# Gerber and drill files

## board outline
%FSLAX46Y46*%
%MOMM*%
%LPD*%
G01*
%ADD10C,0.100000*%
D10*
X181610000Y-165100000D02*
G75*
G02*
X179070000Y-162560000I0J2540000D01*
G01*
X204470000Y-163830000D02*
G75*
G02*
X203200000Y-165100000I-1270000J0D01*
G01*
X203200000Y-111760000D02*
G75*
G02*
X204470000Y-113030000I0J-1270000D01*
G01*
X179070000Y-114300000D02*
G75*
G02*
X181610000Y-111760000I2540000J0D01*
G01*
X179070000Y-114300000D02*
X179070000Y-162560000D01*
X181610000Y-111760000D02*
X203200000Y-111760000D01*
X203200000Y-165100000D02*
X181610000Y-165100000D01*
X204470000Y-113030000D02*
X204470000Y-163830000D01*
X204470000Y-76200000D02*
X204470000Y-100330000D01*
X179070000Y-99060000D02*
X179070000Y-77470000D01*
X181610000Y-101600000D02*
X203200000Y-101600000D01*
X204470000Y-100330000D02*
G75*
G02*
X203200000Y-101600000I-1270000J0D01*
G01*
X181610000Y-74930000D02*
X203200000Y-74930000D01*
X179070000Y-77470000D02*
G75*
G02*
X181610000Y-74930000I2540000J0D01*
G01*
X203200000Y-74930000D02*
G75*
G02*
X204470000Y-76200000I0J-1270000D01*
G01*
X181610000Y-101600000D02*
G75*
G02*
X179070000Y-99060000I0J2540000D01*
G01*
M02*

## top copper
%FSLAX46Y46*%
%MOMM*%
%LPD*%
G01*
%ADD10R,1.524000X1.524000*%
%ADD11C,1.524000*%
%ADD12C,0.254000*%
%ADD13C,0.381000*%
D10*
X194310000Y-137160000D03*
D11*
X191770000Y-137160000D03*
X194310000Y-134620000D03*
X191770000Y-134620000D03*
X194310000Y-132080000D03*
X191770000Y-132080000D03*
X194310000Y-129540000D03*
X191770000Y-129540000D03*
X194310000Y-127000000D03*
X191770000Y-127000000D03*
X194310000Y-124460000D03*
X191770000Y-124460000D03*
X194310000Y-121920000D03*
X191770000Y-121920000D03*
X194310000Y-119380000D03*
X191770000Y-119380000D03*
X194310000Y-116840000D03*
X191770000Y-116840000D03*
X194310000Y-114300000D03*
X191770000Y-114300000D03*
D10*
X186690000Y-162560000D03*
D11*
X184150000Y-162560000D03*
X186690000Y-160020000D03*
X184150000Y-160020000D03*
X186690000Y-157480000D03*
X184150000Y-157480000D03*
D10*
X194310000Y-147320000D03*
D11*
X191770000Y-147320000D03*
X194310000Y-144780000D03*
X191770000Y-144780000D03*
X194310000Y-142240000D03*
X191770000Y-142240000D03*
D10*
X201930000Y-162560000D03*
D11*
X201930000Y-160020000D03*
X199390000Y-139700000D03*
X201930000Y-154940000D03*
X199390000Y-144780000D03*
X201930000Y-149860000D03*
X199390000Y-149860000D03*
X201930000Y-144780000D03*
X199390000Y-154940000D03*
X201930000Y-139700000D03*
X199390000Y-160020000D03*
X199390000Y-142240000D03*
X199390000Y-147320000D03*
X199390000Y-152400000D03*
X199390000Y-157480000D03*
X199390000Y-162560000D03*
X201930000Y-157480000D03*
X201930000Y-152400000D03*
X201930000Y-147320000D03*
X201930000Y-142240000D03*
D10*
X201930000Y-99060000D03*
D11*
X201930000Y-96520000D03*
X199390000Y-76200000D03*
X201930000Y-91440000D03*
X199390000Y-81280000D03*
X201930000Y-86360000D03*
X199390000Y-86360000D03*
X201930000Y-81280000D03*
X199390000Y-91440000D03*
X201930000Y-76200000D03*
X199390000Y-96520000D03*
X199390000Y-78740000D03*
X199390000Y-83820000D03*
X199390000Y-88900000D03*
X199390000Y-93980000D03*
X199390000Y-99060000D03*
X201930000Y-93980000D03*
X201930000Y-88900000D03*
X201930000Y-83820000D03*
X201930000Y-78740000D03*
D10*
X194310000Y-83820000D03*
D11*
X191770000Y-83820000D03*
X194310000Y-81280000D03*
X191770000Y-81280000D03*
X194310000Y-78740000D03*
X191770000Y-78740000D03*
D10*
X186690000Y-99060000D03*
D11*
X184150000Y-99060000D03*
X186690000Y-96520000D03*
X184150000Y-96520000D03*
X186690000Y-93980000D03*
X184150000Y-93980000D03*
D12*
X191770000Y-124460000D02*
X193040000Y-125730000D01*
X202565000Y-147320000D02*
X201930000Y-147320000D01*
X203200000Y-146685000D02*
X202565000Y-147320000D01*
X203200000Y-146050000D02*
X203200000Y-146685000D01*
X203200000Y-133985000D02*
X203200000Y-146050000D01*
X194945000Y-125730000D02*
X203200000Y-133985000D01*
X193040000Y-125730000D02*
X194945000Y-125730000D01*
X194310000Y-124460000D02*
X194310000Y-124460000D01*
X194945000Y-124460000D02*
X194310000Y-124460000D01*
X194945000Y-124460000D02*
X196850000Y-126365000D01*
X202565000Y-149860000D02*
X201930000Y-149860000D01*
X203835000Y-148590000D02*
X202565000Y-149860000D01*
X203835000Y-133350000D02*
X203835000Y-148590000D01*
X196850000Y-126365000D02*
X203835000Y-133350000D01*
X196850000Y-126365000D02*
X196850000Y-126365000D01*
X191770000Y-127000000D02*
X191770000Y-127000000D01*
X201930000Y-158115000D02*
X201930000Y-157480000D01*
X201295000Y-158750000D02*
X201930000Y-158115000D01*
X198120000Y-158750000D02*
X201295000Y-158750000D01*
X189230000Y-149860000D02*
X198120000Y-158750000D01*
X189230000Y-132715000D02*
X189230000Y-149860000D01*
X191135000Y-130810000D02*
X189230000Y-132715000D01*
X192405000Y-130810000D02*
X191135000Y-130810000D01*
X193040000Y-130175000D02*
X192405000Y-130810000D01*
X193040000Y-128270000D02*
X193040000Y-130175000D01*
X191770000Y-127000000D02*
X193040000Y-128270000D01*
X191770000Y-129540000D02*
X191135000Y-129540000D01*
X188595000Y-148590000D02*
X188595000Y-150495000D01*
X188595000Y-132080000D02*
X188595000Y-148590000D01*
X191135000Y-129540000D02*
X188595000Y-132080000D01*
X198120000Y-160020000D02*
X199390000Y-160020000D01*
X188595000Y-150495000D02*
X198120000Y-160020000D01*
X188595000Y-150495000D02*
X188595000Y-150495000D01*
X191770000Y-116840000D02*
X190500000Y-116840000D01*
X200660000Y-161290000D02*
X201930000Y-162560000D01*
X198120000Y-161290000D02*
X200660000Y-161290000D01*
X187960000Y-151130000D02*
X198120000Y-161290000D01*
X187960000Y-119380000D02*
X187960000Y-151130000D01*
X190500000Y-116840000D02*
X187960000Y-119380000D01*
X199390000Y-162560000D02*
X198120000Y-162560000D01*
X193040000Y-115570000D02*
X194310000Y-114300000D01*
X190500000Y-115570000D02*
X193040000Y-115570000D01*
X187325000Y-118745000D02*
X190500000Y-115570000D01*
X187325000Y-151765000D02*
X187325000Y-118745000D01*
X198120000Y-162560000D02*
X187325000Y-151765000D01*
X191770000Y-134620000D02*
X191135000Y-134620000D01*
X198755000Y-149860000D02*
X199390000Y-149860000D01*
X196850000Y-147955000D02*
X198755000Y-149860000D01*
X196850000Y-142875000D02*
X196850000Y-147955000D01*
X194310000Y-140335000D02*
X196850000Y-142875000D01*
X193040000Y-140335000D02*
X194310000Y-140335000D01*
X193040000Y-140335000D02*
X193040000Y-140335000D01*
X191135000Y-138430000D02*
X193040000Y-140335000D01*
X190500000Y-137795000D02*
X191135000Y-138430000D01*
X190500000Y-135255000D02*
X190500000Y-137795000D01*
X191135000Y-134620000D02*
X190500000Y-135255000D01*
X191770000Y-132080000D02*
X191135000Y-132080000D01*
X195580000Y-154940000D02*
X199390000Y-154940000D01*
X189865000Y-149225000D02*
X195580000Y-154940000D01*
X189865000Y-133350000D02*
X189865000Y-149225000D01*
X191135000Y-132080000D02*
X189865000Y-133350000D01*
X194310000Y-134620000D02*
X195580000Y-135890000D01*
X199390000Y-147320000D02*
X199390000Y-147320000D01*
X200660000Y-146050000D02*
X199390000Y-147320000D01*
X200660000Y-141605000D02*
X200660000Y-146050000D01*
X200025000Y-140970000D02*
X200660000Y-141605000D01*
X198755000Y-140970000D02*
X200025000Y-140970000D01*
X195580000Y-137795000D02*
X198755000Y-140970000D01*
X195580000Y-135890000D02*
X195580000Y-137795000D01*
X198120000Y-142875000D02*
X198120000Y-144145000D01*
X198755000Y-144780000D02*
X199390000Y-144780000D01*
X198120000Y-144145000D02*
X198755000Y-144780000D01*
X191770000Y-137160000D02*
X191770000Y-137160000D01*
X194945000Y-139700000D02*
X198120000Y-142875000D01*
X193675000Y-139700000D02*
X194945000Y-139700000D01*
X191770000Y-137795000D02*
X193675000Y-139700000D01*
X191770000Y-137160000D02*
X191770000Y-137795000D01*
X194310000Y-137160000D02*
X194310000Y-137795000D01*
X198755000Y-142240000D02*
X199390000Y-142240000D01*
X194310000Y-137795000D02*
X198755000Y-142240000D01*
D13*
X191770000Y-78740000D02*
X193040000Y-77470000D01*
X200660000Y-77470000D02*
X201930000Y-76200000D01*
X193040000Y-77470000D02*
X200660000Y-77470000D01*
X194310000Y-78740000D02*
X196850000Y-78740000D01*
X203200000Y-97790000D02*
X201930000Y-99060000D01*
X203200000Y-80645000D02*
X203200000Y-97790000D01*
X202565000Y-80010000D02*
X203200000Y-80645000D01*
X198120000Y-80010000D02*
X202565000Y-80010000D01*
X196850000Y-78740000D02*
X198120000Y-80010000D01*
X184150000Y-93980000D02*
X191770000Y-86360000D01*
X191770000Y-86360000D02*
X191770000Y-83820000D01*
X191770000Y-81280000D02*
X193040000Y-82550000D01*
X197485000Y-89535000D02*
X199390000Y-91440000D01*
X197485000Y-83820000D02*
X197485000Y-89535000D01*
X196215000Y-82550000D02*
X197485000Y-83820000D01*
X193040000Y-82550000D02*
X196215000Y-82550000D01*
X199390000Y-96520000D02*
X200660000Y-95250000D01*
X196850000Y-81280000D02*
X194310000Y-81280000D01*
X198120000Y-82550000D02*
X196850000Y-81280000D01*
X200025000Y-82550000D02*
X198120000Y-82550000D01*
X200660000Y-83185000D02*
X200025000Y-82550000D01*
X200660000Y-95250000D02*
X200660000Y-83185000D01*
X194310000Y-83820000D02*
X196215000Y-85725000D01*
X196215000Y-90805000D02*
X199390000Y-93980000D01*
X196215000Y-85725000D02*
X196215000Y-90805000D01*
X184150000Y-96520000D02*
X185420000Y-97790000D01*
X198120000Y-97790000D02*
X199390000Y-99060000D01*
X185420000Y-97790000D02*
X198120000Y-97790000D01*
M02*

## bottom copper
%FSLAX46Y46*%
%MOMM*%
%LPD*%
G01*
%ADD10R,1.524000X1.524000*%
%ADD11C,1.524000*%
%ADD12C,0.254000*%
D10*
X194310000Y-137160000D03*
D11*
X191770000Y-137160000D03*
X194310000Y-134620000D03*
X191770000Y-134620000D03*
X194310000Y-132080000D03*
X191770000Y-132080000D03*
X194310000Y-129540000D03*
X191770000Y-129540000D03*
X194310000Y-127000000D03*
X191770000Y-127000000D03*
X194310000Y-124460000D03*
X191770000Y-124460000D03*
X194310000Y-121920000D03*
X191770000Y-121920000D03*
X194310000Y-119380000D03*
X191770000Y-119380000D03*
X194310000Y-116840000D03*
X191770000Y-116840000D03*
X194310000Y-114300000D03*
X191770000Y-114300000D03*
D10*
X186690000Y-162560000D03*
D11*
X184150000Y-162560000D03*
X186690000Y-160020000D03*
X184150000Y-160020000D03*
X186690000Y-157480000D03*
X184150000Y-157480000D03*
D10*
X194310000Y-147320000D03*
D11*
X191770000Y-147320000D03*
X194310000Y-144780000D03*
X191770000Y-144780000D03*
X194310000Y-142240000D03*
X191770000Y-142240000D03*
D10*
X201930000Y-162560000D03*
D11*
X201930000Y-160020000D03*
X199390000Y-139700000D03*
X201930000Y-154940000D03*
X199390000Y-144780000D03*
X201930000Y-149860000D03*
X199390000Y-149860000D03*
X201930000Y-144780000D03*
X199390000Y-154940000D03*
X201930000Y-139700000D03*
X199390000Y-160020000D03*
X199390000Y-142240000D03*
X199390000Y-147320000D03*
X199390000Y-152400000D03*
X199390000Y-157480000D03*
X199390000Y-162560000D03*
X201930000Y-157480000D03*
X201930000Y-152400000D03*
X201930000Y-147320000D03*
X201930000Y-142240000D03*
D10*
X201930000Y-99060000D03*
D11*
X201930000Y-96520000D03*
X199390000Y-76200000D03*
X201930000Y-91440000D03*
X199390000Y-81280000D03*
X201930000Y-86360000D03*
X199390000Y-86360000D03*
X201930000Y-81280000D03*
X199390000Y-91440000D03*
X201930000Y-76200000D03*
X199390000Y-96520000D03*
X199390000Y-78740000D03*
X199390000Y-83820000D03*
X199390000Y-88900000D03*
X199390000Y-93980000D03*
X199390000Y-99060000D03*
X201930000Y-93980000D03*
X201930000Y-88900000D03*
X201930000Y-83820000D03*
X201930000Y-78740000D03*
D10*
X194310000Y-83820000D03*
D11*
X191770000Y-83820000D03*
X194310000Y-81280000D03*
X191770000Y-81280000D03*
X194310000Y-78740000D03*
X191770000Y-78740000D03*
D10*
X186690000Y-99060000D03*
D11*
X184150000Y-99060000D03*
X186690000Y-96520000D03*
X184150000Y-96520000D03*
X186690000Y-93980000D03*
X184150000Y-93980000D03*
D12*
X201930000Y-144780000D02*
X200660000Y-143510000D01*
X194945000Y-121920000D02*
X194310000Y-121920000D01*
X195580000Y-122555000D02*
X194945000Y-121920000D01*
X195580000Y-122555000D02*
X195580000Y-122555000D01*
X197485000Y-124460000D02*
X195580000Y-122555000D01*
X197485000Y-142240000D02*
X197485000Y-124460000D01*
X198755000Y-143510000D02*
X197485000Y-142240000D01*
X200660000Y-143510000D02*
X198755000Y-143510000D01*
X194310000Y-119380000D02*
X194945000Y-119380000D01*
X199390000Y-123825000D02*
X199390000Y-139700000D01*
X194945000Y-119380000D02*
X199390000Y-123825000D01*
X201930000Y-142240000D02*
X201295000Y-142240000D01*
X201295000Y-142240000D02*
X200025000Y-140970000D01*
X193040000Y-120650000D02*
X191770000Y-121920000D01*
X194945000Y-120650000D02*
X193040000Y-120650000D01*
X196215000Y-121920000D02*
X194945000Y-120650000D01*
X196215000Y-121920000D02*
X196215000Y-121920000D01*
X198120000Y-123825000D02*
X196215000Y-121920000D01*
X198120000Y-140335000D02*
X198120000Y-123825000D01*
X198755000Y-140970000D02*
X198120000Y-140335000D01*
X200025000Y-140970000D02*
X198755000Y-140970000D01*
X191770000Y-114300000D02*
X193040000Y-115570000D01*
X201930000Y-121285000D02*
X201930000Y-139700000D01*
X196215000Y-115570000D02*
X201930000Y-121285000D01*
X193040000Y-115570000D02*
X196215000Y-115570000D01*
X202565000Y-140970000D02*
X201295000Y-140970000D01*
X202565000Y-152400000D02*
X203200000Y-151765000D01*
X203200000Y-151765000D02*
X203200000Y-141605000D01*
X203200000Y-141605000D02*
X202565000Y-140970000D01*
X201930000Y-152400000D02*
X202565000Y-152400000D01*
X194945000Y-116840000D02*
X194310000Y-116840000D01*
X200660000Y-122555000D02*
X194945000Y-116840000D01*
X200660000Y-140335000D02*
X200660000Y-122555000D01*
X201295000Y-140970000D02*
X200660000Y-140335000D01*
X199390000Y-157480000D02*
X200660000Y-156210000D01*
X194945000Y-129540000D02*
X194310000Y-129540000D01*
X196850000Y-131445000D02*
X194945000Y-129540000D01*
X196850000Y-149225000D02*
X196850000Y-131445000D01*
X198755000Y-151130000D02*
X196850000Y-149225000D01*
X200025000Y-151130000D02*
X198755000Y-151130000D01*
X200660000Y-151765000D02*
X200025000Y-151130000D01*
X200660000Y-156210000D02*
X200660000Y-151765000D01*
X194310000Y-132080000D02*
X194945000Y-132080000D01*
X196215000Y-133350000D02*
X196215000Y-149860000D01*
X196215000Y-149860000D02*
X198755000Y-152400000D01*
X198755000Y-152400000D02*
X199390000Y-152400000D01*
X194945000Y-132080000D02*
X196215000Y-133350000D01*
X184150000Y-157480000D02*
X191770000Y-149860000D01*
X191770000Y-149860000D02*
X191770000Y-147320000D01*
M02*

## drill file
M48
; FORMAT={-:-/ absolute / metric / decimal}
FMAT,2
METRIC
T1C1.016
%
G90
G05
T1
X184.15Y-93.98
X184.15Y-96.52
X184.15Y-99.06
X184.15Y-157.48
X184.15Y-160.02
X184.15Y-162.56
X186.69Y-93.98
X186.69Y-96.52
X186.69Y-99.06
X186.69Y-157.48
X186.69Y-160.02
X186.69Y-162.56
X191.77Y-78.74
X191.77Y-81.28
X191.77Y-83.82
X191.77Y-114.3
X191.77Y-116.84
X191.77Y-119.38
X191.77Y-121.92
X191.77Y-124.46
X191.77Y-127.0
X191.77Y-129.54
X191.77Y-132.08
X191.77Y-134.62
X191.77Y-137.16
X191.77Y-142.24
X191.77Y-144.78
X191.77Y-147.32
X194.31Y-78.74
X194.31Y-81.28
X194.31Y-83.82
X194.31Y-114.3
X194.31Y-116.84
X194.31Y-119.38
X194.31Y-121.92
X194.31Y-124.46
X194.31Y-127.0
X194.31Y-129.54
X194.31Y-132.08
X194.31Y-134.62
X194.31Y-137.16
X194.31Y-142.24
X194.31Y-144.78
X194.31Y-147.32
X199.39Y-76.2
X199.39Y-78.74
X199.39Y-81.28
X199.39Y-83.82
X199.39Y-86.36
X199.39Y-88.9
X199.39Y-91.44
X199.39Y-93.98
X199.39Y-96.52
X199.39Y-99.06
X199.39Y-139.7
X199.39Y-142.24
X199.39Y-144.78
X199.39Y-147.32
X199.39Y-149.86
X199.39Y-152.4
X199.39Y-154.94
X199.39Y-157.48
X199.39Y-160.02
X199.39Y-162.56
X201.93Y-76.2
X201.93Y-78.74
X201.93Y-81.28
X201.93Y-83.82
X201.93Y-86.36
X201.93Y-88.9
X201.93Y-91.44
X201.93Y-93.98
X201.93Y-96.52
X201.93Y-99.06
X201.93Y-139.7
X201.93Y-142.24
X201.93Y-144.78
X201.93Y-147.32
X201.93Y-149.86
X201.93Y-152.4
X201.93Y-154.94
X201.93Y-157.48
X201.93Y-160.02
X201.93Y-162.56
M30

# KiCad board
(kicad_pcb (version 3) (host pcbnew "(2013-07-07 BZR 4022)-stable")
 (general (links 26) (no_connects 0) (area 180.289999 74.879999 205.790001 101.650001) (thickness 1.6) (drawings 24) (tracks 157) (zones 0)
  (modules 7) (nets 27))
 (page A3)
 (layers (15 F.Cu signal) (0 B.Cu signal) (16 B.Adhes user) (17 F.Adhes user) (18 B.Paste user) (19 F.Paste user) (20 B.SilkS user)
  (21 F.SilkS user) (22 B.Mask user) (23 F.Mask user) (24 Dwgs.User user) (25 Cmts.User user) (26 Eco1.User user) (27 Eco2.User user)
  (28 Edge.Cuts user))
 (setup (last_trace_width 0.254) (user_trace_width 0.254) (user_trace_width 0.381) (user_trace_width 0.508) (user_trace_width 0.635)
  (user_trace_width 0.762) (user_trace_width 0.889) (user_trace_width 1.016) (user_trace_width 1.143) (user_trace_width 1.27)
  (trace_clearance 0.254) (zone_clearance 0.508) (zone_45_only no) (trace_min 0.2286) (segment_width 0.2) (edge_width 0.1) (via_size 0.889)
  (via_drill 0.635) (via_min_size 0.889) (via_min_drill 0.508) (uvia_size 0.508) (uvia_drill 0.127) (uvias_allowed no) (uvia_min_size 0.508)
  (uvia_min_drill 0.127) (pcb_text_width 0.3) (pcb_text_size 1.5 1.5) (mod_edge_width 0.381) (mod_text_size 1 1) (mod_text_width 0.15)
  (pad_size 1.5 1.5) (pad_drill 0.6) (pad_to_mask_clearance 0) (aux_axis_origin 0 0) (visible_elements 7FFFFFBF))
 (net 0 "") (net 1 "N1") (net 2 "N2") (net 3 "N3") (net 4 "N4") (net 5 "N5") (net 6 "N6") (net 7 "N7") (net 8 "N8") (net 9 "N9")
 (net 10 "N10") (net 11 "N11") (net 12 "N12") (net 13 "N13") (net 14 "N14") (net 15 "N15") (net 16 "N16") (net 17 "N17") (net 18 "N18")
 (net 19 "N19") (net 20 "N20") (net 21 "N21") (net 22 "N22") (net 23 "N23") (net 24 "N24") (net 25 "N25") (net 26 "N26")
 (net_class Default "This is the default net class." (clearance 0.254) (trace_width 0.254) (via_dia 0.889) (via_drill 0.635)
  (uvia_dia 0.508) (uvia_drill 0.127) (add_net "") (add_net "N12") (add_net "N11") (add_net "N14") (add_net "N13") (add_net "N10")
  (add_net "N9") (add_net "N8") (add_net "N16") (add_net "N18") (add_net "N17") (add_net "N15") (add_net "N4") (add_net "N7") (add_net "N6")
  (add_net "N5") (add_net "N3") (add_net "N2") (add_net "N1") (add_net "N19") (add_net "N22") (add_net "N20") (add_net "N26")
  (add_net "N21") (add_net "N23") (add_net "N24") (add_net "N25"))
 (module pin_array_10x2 (layer F.Cu) (at 193.04 125.73 90)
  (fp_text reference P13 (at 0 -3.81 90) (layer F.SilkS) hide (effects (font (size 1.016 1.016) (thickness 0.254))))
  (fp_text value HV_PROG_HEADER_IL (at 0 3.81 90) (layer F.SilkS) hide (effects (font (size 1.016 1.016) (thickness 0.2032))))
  (pad 1 thru_hole rect (at -11.43 1.27 90) (size 1.524 1.524) (drill 1.016) (layers *.Cu *.Mask F.SilkS) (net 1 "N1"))
  (pad 2 thru_hole circle (at -11.43 -1.27 90) (size 1.524 1.524) (drill 1.016) (layers *.Cu *.Mask F.SilkS) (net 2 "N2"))
  (pad 3 thru_hole circle (at -8.89 1.27 90) (size 1.524 1.524) (drill 1.016) (layers *.Cu *.Mask F.SilkS) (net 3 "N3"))
  (pad 4 thru_hole circle (at -8.89 -1.27 90) (size 1.524 1.524) (drill 1.016) (layers *.Cu *.Mask F.SilkS) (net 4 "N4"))
  (pad 5 thru_hole circle (at -6.35 1.27 90) (size 1.524 1.524) (drill 1.016) (layers *.Cu *.Mask F.SilkS) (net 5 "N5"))
  (pad 6 thru_hole circle (at -6.35 -1.27 90) (size 1.524 1.524) (drill 1.016) (layers *.Cu *.Mask F.SilkS) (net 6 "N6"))
  (pad 7 thru_hole circle (at -3.81 1.27 90) (size 1.524 1.524) (drill 1.016) (layers *.Cu *.Mask F.SilkS) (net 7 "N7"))
  (pad 8 thru_hole circle (at -3.81 -1.27 90) (size 1.524 1.524) (drill 1.016) (layers *.Cu *.Mask F.SilkS) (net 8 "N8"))
  (pad 9 thru_hole circle (at -1.27 1.27 90) (size 1.524 1.524) (drill 1.016) (layers *.Cu *.Mask F.SilkS))
  (pad 10 thru_hole circle (at -1.27 -1.27 90) (size 1.524 1.524) (drill 1.016) (layers *.Cu *.Mask F.SilkS) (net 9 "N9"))
  (pad 11 thru_hole circle (at 1.27 1.27 90) (size 1.524 1.524) (drill 1.016) (layers *.Cu *.Mask F.SilkS) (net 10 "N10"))
  (pad 12 thru_hole circle (at 1.27 -1.27 90) (size 1.524 1.524) (drill 1.016) (layers *.Cu *.Mask F.SilkS) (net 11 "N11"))
  (pad 13 thru_hole circle (at 3.81 1.27 90) (size 1.524 1.524) (drill 1.016) (layers *.Cu *.Mask F.SilkS) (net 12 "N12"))
  (pad 14 thru_hole circle (at 3.81 -1.27 90) (size 1.524 1.524) (drill 1.016) (layers *.Cu *.Mask F.SilkS) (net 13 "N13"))
  (pad 15 thru_hole circle (at 6.35 1.27 90) (size 1.524 1.524) (drill 1.016) (layers *.Cu *.Mask F.SilkS) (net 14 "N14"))
  (pad 16 thru_hole circle (at 6.35 -1.27 90) (size 1.524 1.524) (drill 1.016) (layers *.Cu *.Mask F.SilkS))
  (pad 17 thru_hole circle (at 8.89 1.27 90) (size 1.524 1.524) (drill 1.016) (layers *.Cu *.Mask F.SilkS) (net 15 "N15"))
  (pad 18 thru_hole circle (at 8.89 -1.27 90) (size 1.524 1.524) (drill 1.016) (layers *.Cu *.Mask F.SilkS) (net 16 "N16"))
  (pad 19 thru_hole circle (at 11.43 1.27 90) (size 1.524 1.524) (drill 1.016) (layers *.Cu *.Mask F.SilkS) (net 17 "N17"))
  (pad 20 thru_hole circle (at 11.43 -1.27 90) (size 1.524 1.524) (drill 1.016) (layers *.Cu *.Mask F.SilkS) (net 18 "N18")))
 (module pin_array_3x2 (layer F.Cu) (at 185.42 160.02 90)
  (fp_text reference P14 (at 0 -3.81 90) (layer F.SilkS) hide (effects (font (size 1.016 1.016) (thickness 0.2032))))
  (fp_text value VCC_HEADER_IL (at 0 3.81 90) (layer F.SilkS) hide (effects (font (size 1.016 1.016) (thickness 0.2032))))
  (pad 1 thru_hole rect (at -2.54 1.27 90) (size 1.524 1.524) (drill 1.016) (layers *.Cu *.Mask F.SilkS))
  (pad 2 thru_hole circle (at -2.54 -1.27 90) (size 1.524 1.524) (drill 1.016) (layers *.Cu *.Mask F.SilkS))
  (pad 3 thru_hole circle (at 0 1.27 90) (size 1.524 1.524) (drill 1.016) (layers *.Cu *.Mask F.SilkS))
  (pad 4 thru_hole circle (at 0 -1.27 90) (size 1.524 1.524) (drill 1.016) (layers *.Cu *.Mask F.SilkS))
  (pad 5 thru_hole circle (at 2.54 1.27 90) (size 1.524 1.524) (drill 1.016) (layers *.Cu *.Mask F.SilkS))
  (pad 6 thru_hole circle (at 2.54 -1.27 90) (size 1.524 1.524) (drill 1.016) (layers *.Cu *.Mask F.SilkS) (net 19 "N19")))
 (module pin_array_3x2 (layer F.Cu) (at 193.04 144.78 90)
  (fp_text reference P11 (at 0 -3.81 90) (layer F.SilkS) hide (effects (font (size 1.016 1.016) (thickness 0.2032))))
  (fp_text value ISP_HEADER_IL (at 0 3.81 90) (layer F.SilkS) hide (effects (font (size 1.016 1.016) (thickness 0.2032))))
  (pad 1 thru_hole rect (at -2.54 1.27 90) (size 1.524 1.524) (drill 1.016) (layers *.Cu *.Mask F.SilkS))
  (pad 2 thru_hole circle (at -2.54 -1.27 90) (size 1.524 1.524) (drill 1.016) (layers *.Cu *.Mask F.SilkS) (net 19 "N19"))
  (pad 3 thru_hole circle (at 0 1.27 90) (size 1.524 1.524) (drill 1.016) (layers *.Cu *.Mask F.SilkS))
  (pad 4 thru_hole circle (at 0 -1.27 90) (size 1.524 1.524) (drill 1.016) (layers *.Cu *.Mask F.SilkS))
  (pad 5 thru_hole circle (at 2.54 1.27 90) (size 1.524 1.524) (drill 1.016) (layers *.Cu *.Mask F.SilkS))
  (pad 6 thru_hole circle (at 2.54 -1.27 90) (size 1.524 1.524) (drill 1.016) (layers *.Cu *.Mask F.SilkS)))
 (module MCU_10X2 (layer F.Cu) (at 200.66 151.13 90)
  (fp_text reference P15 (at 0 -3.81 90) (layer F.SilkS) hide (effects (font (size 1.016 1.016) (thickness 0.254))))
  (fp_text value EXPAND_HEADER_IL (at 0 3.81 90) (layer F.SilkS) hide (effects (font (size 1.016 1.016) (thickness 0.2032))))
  (pad 1 thru_hole rect (at -11.43 1.27 90) (size 1.524 1.524) (drill 1.016) (layers *.Cu *.Mask F.SilkS) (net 16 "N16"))
  (pad 2 thru_hole circle (at -8.89 1.27 90) (size 1.524 1.524) (drill 1.016) (layers *.Cu *.Mask F.SilkS))
  (pad 11 thru_hole circle (at 11.43 -1.27 90) (size 1.524 1.524) (drill 1.016) (layers *.Cu *.Mask F.SilkS) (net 14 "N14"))
  (pad 4 thru_hole circle (at -3.81 1.27 90) (size 1.524 1.524) (drill 1.016) (layers *.Cu *.Mask F.SilkS))
  (pad 13 thru_hole circle (at 6.35 -1.27 90) (size 1.524 1.524) (drill 1.016) (layers *.Cu *.Mask F.SilkS) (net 2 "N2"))
  (pad 6 thru_hole circle (at 1.27 1.27 90) (size 1.524 1.524) (drill 1.016) (layers *.Cu *.Mask F.SilkS) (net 10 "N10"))
  (pad 15 thru_hole circle (at 1.27 -1.27 90) (size 1.524 1.524) (drill 1.016) (layers *.Cu *.Mask F.SilkS) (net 4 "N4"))
  (pad 8 thru_hole circle (at 6.35 1.27 90) (size 1.524 1.524) (drill 1.016) (layers *.Cu *.Mask F.SilkS) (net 12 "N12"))
  (pad 17 thru_hole circle (at -3.81 -1.27 90) (size 1.524 1.524) (drill 1.016) (layers *.Cu *.Mask F.SilkS) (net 6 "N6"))
  (pad 10 thru_hole circle (at 11.43 1.27 90) (size 1.524 1.524) (drill 1.016) (layers *.Cu *.Mask F.SilkS) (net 18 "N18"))
  (pad 19 thru_hole circle (at -8.89 -1.27 90) (size 1.524 1.524) (drill 1.016) (layers *.Cu *.Mask F.SilkS) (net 8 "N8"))
  (pad 12 thru_hole circle (at 8.89 -1.27 90) (size 1.524 1.524) (drill 1.016) (layers *.Cu *.Mask F.SilkS) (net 1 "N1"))
  (pad 14 thru_hole circle (at 3.81 -1.27 90) (size 1.524 1.524) (drill 1.016) (layers *.Cu *.Mask F.SilkS) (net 3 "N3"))
  (pad 16 thru_hole circle (at -1.27 -1.27 90) (size 1.524 1.524) (drill 1.016) (layers *.Cu *.Mask F.SilkS) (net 5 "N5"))
  (pad 18 thru_hole circle (at -6.35 -1.27 90) (size 1.524 1.524) (drill 1.016) (layers *.Cu *.Mask F.SilkS) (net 7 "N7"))
  (pad 20 thru_hole circle (at -11.43 -1.27 90) (size 1.524 1.524) (drill 1.016) (layers *.Cu *.Mask F.SilkS) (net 17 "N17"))
  (pad 3 thru_hole circle (at -6.35 1.27 90) (size 1.524 1.524) (drill 1.016) (layers *.Cu *.Mask F.SilkS) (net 9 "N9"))
  (pad 5 thru_hole circle (at -1.27 1.27 90) (size 1.524 1.524) (drill 1.016) (layers *.Cu *.Mask F.SilkS) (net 15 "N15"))
  (pad 7 thru_hole circle (at 3.81 1.27 90) (size 1.524 1.524) (drill 1.016) (layers *.Cu *.Mask F.SilkS) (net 11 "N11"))
  (pad 9 thru_hole circle (at 8.89 1.27 90) (size 1.524 1.524) (drill 1.016) (layers *.Cu *.Mask F.SilkS) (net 13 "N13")))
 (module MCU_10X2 (layer F.Cu) (at 200.66 87.63 90)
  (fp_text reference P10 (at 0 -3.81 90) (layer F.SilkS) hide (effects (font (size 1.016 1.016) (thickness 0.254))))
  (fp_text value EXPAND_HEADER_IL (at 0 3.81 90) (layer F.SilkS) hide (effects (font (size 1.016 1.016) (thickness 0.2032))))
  (pad 1 thru_hole rect (at -11.43 1.27 90) (size 1.524 1.524) (drill 1.016) (layers *.Cu *.Mask F.SilkS) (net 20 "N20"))
  (pad 2 thru_hole circle (at -8.89 1.27 90) (size 1.524 1.524) (drill 1.016) (layers *.Cu *.Mask F.SilkS))
  (pad 11 thru_hole circle (at 11.43 -1.27 90) (size 1.524 1.524) (drill 1.016) (layers *.Cu *.Mask F.SilkS))
  (pad 4 thru_hole circle (at -3.81 1.27 90) (size 1.524 1.524) (drill 1.016) (layers *.Cu *.Mask F.SilkS))
  (pad 13 thru_hole circle (at 6.35 -1.27 90) (size 1.524 1.524) (drill 1.016) (layers *.Cu *.Mask F.SilkS))
  (pad 6 thru_hole circle (at 1.27 1.27 90) (size 1.524 1.524) (drill 1.016) (layers *.Cu *.Mask F.SilkS))
  (pad 15 thru_hole circle (at 1.27 -1.27 90) (size 1.524 1.524) (drill 1.016) (layers *.Cu *.Mask F.SilkS))
  (pad 8 thru_hole circle (at 6.35 1.27 90) (size 1.524 1.524) (drill 1.016) (layers *.Cu *.Mask F.SilkS))
  (pad 17 thru_hole circle (at -3.81 -1.27 90) (size 1.524 1.524) (drill 1.016) (layers *.Cu *.Mask F.SilkS) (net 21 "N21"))
  (pad 10 thru_hole circle (at 11.43 1.27 90) (size 1.524 1.524) (drill 1.016) (layers *.Cu *.Mask F.SilkS) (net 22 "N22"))
  (pad 19 thru_hole circle (at -8.89 -1.27 90) (size 1.524 1.524) (drill 1.016) (layers *.Cu *.Mask F.SilkS) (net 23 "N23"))
  (pad 12 thru_hole circle (at 8.89 -1.27 90) (size 1.524 1.524) (drill 1.016) (layers *.Cu *.Mask F.SilkS))
  (pad 14 thru_hole circle (at 3.81 -1.27 90) (size 1.524 1.524) (drill 1.016) (layers *.Cu *.Mask F.SilkS))
  (pad 16 thru_hole circle (at -1.27 -1.27 90) (size 1.524 1.524) (drill 1.016) (layers *.Cu *.Mask F.SilkS))
  (pad 18 thru_hole circle (at -6.35 -1.27 90) (size 1.524 1.524) (drill 1.016) (layers *.Cu *.Mask F.SilkS) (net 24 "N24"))
  (pad 20 thru_hole circle (at -11.43 -1.27 90) (size 1.524 1.524) (drill 1.016) (layers *.Cu *.Mask F.SilkS) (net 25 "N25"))
  (pad 3 thru_hole circle (at -6.35 1.27 90) (size 1.524 1.524) (drill 1.016) (layers *.Cu *.Mask F.SilkS))
  (pad 5 thru_hole circle (at -1.27 1.27 90) (size 1.524 1.524) (drill 1.016) (layers *.Cu *.Mask F.SilkS))
  (pad 7 thru_hole circle (at 3.81 1.27 90) (size 1.524 1.524) (drill 1.016) (layers *.Cu *.Mask F.SilkS))
  (pad 9 thru_hole circle (at 8.89 1.27 90) (size 1.524 1.524) (drill 1.016) (layers *.Cu *.Mask F.SilkS)))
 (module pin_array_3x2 (layer F.Cu) (at 193.04 81.28 90)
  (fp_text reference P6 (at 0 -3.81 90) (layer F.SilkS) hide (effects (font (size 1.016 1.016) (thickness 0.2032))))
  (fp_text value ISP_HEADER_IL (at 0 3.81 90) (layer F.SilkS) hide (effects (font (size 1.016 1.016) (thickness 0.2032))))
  (pad 1 thru_hole rect (at -2.54 1.27 90) (size 1.524 1.524) (drill 1.016) (layers *.Cu *.Mask F.SilkS) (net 24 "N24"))
  (pad 2 thru_hole circle (at -2.54 -1.27 90) (size 1.524 1.524) (drill 1.016) (layers *.Cu *.Mask F.SilkS) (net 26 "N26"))
  (pad 3 thru_hole circle (at 0 1.27 90) (size 1.524 1.524) (drill 1.016) (layers *.Cu *.Mask F.SilkS) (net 23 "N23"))
  (pad 4 thru_hole circle (at 0 -1.27 90) (size 1.524 1.524) (drill 1.016) (layers *.Cu *.Mask F.SilkS) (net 21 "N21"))
  (pad 5 thru_hole circle (at 2.54 1.27 90) (size 1.524 1.524) (drill 1.016) (layers *.Cu *.Mask F.SilkS) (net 20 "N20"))
  (pad 6 thru_hole circle (at 2.54 -1.27 90) (size 1.524 1.524) (drill 1.016) (layers *.Cu *.Mask F.SilkS) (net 22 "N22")))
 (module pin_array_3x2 (layer F.Cu) (at 185.42 96.52 90)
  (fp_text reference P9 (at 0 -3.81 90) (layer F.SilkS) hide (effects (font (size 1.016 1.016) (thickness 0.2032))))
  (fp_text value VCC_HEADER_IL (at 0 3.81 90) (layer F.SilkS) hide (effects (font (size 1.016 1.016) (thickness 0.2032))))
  (pad 1 thru_hole rect (at -2.54 1.27 90) (size 1.524 1.524) (drill 1.016) (layers *.Cu *.Mask F.SilkS))
  (pad 2 thru_hole circle (at -2.54 -1.27 90) (size 1.524 1.524) (drill 1.016) (layers *.Cu *.Mask F.SilkS))
  (pad 3 thru_hole circle (at 0 1.27 90) (size 1.524 1.524) (drill 1.016) (layers *.Cu *.Mask F.SilkS))
  (pad 4 thru_hole circle (at 0 -1.27 90) (size 1.524 1.524) (drill 1.016) (layers *.Cu *.Mask F.SilkS) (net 25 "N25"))
  (pad 5 thru_hole circle (at 2.54 1.27 90) (size 1.524 1.524) (drill 1.016) (layers *.Cu *.Mask F.SilkS))
  (pad 6 thru_hole circle (at 2.54 -1.27 90) (size 1.524 1.524) (drill 1.016) (layers *.Cu *.Mask F.SilkS) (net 26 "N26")))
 (gr_arc (start 181.61 162.56) (end 181.61 165.1) (angle 90) (layer Edge.Cuts) (width 0.1))
 (gr_arc (start 203.2 163.83) (end 204.47 163.83) (angle 90) (layer Edge.Cuts) (width 0.1))
 (gr_arc (start 203.2 113.03) (end 203.2 111.76) (angle 90) (layer Edge.Cuts) (width 0.1))
 (gr_arc (start 181.61 114.3) (end 179.07 114.3) (angle 90) (layer Edge.Cuts) (width 0.1))
 (gr_line (start 179.07 114.3) (end 179.07 162.56) (angle 90) (layer Edge.Cuts) (width 0.1))
 (gr_line (start 181.61 111.76) (end 203.2 111.76) (angle 90) (layer Edge.Cuts) (width 0.1))
 (gr_line (start 203.2 165.1) (end 181.61 165.1) (angle 90) (layer Edge.Cuts) (width 0.1))
 (gr_line (start 204.47 113.03) (end 204.47 163.83) (angle 90) (layer Edge.Cuts) (width 0.1))
 (gr_line (start 204.47 76.2) (end 204.47 100.33) (angle 90) (layer Edge.Cuts) (width 0.1))
 (gr_line (start 179.07 99.06) (end 179.07 77.47) (angle 90) (layer Edge.Cuts) (width 0.1))
 (gr_line (start 181.61 101.6) (end 203.2 101.6) (angle 90) (layer Edge.Cuts) (width 0.1))
 (gr_arc (start 203.2 100.33) (end 204.47 100.33) (angle 90) (layer Edge.Cuts) (width 0.1))
 (gr_line (start 181.61 74.93) (end 203.2 74.93) (angle 90) (layer Edge.Cuts) (width 0.1))
 (gr_arc (start 181.61 77.47) (end 179.07 77.47) (angle 90) (layer Edge.Cuts) (width 0.1))
 (gr_arc (start 203.2 76.2) (end 203.2 74.93) (angle 90) (layer Edge.Cuts) (width 0.1))
 (gr_arc (start 181.61 99.06) (end 181.61 101.6) (angle 90) (layer Edge.Cuts) (width 0.1))
 (segment (start 201.93 144.78) (end 200.66 143.51) (width 0.254) (layer B.Cu) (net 12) (status 400000))
 (segment (start 194.945 121.92) (end 194.31 121.92) (width 0.254) (layer B.Cu) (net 12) (status C00000))
 (segment (start 195.58 122.555) (end 194.945 121.92) (width 0.254) (layer B.Cu) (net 12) (status 800000))
 (segment (start 195.58 122.555) (end 195.58 122.555) (width 0.254) (layer B.Cu) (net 12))
 (segment (start 197.485 124.46) (end 195.58 122.555) (width 0.254) (layer B.Cu) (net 12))
 (segment (start 197.485 142.24) (end 197.485 124.46) (width 0.254) (layer B.Cu) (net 12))
 (segment (start 198.755 143.51) (end 197.485 142.24) (width 0.254) (layer B.Cu) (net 12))
 (segment (start 200.66 143.51) (end 198.755 143.51) (width 0.254) (layer B.Cu) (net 12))
 (segment (start 191.77 124.46) (end 193.04 125.73) (width 0.254) (layer F.Cu) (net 11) (status 400000))
 (segment (start 202.565 147.32) (end 201.93 147.32) (width 0.254) (layer F.Cu) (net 11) (status C00000))
 (segment (start 203.2 146.685) (end 202.565 147.32) (width 0.254) (layer F.Cu) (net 11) (status 800000))
 (segment (start 203.2 146.05) (end 203.2 146.685) (width 0.254) (layer F.Cu) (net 11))
 (segment (start 203.2 133.985) (end 203.2 146.05) (width 0.254) (layer F.Cu) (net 11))
 (segment (start 194.945 125.73) (end 203.2 133.985) (width 0.254) (layer F.Cu) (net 11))
 (segment (start 193.04 125.73) (end 194.945 125.73) (width 0.254) (layer F.Cu) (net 11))
 (segment (start 194.31 119.38) (end 194.945 119.38) (width 0.254) (layer B.Cu) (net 14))
 (segment (start 199.39 123.825) (end 199.39 139.7) (width 0.254) (layer B.Cu) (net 14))
 (segment (start 194.945 119.38) (end 199.39 123.825) (width 0.254) (layer B.Cu) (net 14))
 (segment (start 201.93 142.24) (end 201.295 142.24) (width 0.254) (layer B.Cu) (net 13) (status C00000))
 (segment (start 201.295 142.24) (end 200.025 140.97) (width 0.254) (layer B.Cu) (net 13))
 (segment (start 193.04 120.65) (end 191.77 121.92) (width 0.254) (layer B.Cu) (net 13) (status 800000))
 (segment (start 194.945 120.65) (end 193.04 120.65) (width 0.254) (layer B.Cu) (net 13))
 (segment (start 196.215 121.92) (end 194.945 120.65) (width 0.254) (layer B.Cu) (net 13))
 (segment (start 196.215 121.92) (end 196.215 121.92) (width 0.254) (layer B.Cu) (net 13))
 (segment (start 198.12 123.825) (end 196.215 121.92) (width 0.254) (layer B.Cu) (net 13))
 (segment (start 198.12 140.335) (end 198.12 123.825) (width 0.254) (layer B.Cu) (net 13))
 (segment (start 198.755 140.97) (end 198.12 140.335) (width 0.254) (layer B.Cu) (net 13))
 (segment (start 200.025 140.97) (end 198.755 140.97) (width 0.254) (layer B.Cu) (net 13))
 (segment (start 194.31 124.46) (end 194.31 124.46) (width 0.254) (layer F.Cu) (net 10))
 (segment (start 194.945 124.46) (end 194.31 124.46) (width 0.254) (layer F.Cu) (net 10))
 (segment (start 194.945 124.46) (end 196.85 126.365) (width 0.254) (layer F.Cu) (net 10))
 (segment (start 202.565 149.86) (end 201.93 149.86) (width 0.254) (layer F.Cu) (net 10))
 (segment (start 203.835 148.59) (end 202.565 149.86) (width 0.254) (layer F.Cu) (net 10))
 (segment (start 203.835 133.35) (end 203.835 148.59) (width 0.254) (layer F.Cu) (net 10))
 (segment (start 196.85 126.365) (end 203.835 133.35) (width 0.254) (layer F.Cu) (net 10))
 (segment (start 196.85 126.365) (end 196.85 126.365) (width 0.254) (layer F.Cu) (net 10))
 (segment (start 191.77 127) (end 191.77 127) (width 0.254) (layer F.Cu) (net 9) (status C00000))
 (segment (start 201.93 158.115) (end 201.93 157.48) (width 0.254) (layer F.Cu) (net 9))
 (segment (start 201.295 158.75) (end 201.93 158.115) (width 0.254) (layer F.Cu) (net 9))
 (segment (start 198.12 158.75) (end 201.295 158.75) (width 0.254) (layer F.Cu) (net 9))
 (segment (start 189.23 149.86) (end 198.12 158.75) (width 0.254) (layer F.Cu) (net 9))
 (segment (start 189.23 132.715) (end 189.23 149.86) (width 0.254) (layer F.Cu) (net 9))
 (segment (start 191.135 130.81) (end 189.23 132.715) (width 0.254) (layer F.Cu) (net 9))
 (segment (start 192.405 130.81) (end 191.135 130.81) (width 0.254) (layer F.Cu) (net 9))
 (segment (start 193.04 130.175) (end 192.405 130.81) (width 0.254) (layer F.Cu) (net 9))
 (segment (start 193.04 128.27) (end 193.04 130.175) (width 0.254) (layer F.Cu) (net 9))
 (segment (start 191.77 127) (end 193.04 128.27) (width 0.254) (layer F.Cu) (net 9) (status 400000))
 (segment (start 191.77 129.54) (end 191.135 129.54) (width 0.254) (layer F.Cu) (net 8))
 (segment (start 188.595 148.59) (end 188.595 150.495) (width 0.254) (layer F.Cu) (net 8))
 (segment (start 188.595 132.08) (end 188.595 148.59) (width 0.254) (layer F.Cu) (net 8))
 (segment (start 191.135 129.54) (end 188.595 132.08) (width 0.254) (layer F.Cu) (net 8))
 (segment (start 198.12 160.02) (end 199.39 160.02) (width 0.254) (layer F.Cu) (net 8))
 (segment (start 188.595 150.495) (end 198.12 160.02) (width 0.254) (layer F.Cu) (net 8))
 (segment (start 188.595 150.495) (end 188.595 150.495) (width 0.254) (layer F.Cu) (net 8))
 (segment (start 191.77 116.84) (end 190.5 116.84) (width 0.254) (layer F.Cu) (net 16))
 (segment (start 200.66 161.29) (end 201.93 162.56) (width 0.254) (layer F.Cu) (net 16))
 (segment (start 198.12 161.29) (end 200.66 161.29) (width 0.254) (layer F.Cu) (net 16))
 (segment (start 187.96 151.13) (end 198.12 161.29) (width 0.254) (layer F.Cu) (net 16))
 (segment (start 187.96 119.38) (end 187.96 151.13) (width 0.254) (layer F.Cu) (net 16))
 (segment (start 190.5 116.84) (end 187.96 119.38) (width 0.254) (layer F.Cu) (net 16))
 (segment (start 191.77 114.3) (end 193.04 115.57) (width 0.254) (layer B.Cu) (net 18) (status 400000))
 (segment (start 201.93 121.285) (end 201.93 139.7) (width 0.254) (layer B.Cu) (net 18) (status 800000))
 (segment (start 196.215 115.57) (end 201.93 121.285) (width 0.254) (layer B.Cu) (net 18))
 (segment (start 193.04 115.57) (end 196.215 115.57) (width 0.254) (layer B.Cu) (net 18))
 (segment (start 199.39 162.56) (end 198.12 162.56) (width 0.254) (layer F.Cu) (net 17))
 (segment (start 193.04 115.57) (end 194.31 114.3) (width 0.254) (layer F.Cu) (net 17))
 (segment (start 190.5 115.57) (end 193.04 115.57) (width 0.254) (layer F.Cu) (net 17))
 (segment (start 187.325 118.745) (end 190.5 115.57) (width 0.254) (layer F.Cu) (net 17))
 (segment (start 187.325 151.765) (end 187.325 118.745) (width 0.254) (layer F.Cu) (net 17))
 (segment (start 198.12 162.56) (end 187.325 151.765) (width 0.254) (layer F.Cu) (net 17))
 (segment (start 202.565 140.97) (end 201.295 140.97) (width 0.254) (layer B.Cu) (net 15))
 (segment (start 202.565 152.4) (end 203.2 151.765) (width 0.254) (layer B.Cu) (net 15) (status 400000))
 (segment (start 203.2 151.765) (end 203.2 141.605) (width 0.254) (layer B.Cu) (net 15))
 (segment (start 203.2 141.605) (end 202.565 140.97) (width 0.254) (layer B.Cu) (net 15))
 (segment (start 201.93 152.4) (end 202.565 152.4) (width 0.254) (layer B.Cu) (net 15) (status C00000))
 (segment (start 194.945 116.84) (end 194.31 116.84) (width 0.254) (layer B.Cu) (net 15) (status C00000))
 (segment (start 200.66 122.555) (end 194.945 116.84) (width 0.254) (layer B.Cu) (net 15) (status 800000))
 (segment (start 200.66 140.335) (end 200.66 122.555) (width 0.254) (layer B.Cu) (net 15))
 (segment (start 201.295 140.97) (end 200.66 140.335) (width 0.254) (layer B.Cu) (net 15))
 (segment (start 191.77 134.62) (end 191.135 134.62) (width 0.254) (layer F.Cu) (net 4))
 (segment (start 198.755 149.86) (end 199.39 149.86) (width 0.254) (layer F.Cu) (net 4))
 (segment (start 196.85 147.955) (end 198.755 149.86) (width 0.254) (layer F.Cu) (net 4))
 (segment (start 196.85 142.875) (end 196.85 147.955) (width 0.254) (layer F.Cu) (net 4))
 (segment (start 194.31 140.335) (end 196.85 142.875) (width 0.254) (layer F.Cu) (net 4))
 (segment (start 193.04 140.335) (end 194.31 140.335) (width 0.254) (layer F.Cu) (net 4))
 (segment (start 193.04 140.335) (end 193.04 140.335) (width 0.254) (layer F.Cu) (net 4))
 (segment (start 191.135 138.43) (end 193.04 140.335) (width 0.254) (layer F.Cu) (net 4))
 (segment (start 190.5 137.795) (end 191.135 138.43) (width 0.254) (layer F.Cu) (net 4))
 (segment (start 190.5 135.255) (end 190.5 137.795) (width 0.254) (layer F.Cu) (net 4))
 (segment (start 191.135 134.62) (end 190.5 135.255) (width 0.254) (layer F.Cu) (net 4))
 (segment (start 199.39 157.48) (end 200.66 156.21) (width 0.254) (layer B.Cu) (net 7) (status 400000))
 (segment (start 194.945 129.54) (end 194.31 129.54) (width 0.254) (layer B.Cu) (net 7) (status C00000))
 (segment (start 196.85 131.445) (end 194.945 129.54) (width 0.254) (layer B.Cu) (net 7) (status 800000))
 (segment (start 196.85 149.225) (end 196.85 131.445) (width 0.254) (layer B.Cu) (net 7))
 (segment (start 198.755 151.13) (end 196.85 149.225) (width 0.254) (layer B.Cu) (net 7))
 (segment (start 200.025 151.13) (end 198.755 151.13) (width 0.254) (layer B.Cu) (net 7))
 (segment (start 200.66 151.765) (end 200.025 151.13) (width 0.254) (layer B.Cu) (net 7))
 (segment (start 200.66 156.21) (end 200.66 151.765) (width 0.254) (layer B.Cu) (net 7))
 (segment (start 191.77 132.08) (end 191.135 132.08) (width 0.254) (layer F.Cu) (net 6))
 (segment (start 195.58 154.94) (end 199.39 154.94) (width 0.254) (layer F.Cu) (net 6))
 (segment (start 189.865 149.225) (end 195.58 154.94) (width 0.254) (layer F.Cu) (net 6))
 (segment (start 189.865 133.35) (end 189.865 149.225) (width 0.254) (layer F.Cu) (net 6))
 (segment (start 191.135 132.08) (end 189.865 133.35) (width 0.254) (layer F.Cu) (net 6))
 (segment (start 194.31 132.08) (end 194.945 132.08) (width 0.254) (layer B.Cu) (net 5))
 (segment (start 196.215 133.35) (end 196.215 149.86) (width 0.254) (layer B.Cu) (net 5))
 (segment (start 196.215 149.86) (end 198.755 152.4) (width 0.254) (layer B.Cu) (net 5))
 (segment (start 198.755 152.4) (end 199.39 152.4) (width 0.254) (layer B.Cu) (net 5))
 (segment (start 194.945 132.08) (end 196.215 133.35) (width 0.254) (layer B.Cu) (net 5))
 (segment (start 194.31 134.62) (end 195.58 135.89) (width 0.254) (layer F.Cu) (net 3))
 (segment (start 199.39 147.32) (end 199.39 147.32) (width 0.254) (layer F.Cu) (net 3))
 (segment (start 200.66 146.05) (end 199.39 147.32) (width 0.254) (layer F.Cu) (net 3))
 (segment (start 200.66 141.605) (end 200.66 146.05) (width 0.254) (layer F.Cu) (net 3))
 (segment (start 200.025 140.97) (end 200.66 141.605) (width 0.254) (layer F.Cu) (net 3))
 (segment (start 198.755 140.97) (end 200.025 140.97) (width 0.254) (layer F.Cu) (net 3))
 (segment (start 195.58 137.795) (end 198.755 140.97) (width 0.254) (layer F.Cu) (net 3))
 (segment (start 195.58 135.89) (end 195.58 137.795) (width 0.254) (layer F.Cu) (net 3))
 (segment (start 198.12 142.875) (end 198.12 144.145) (width 0.254) (layer F.Cu) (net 2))
 (segment (start 198.755 144.78) (end 199.39 144.78) (width 0.254) (layer F.Cu) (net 2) (status C00000))
 (segment (start 198.12 144.145) (end 198.755 144.78) (width 0.254) (layer F.Cu) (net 2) (status 800000))
 (segment (start 191.77 137.16) (end 191.77 137.16) (width 0.254) (layer F.Cu) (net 2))
 (segment (start 194.945 139.7) (end 198.12 142.875) (width 0.254) (layer F.Cu) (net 2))
 (segment (start 193.675 139.7) (end 194.945 139.7) (width 0.254) (layer F.Cu) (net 2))
 (segment (start 191.77 137.795) (end 193.675 139.7) (width 0.254) (layer F.Cu) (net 2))
 (segment (start 191.77 137.16) (end 191.77 137.795) (width 0.254) (layer F.Cu) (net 2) (status 400000))
 (segment (start 194.31 137.16) (end 194.31 137.795) (width 0.254) (layer F.Cu) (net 1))
 (segment (start 198.755 142.24) (end 199.39 142.24) (width 0.254) (layer F.Cu) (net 1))
 (segment (start 194.31 137.795) (end 198.755 142.24) (width 0.254) (layer F.Cu) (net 1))
 (segment (start 184.15 157.48) (end 191.77 149.86) (width 0.254) (layer B.Cu) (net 19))
 (segment (start 191.77 149.86) (end 191.77 147.32) (width 0.254) (layer B.Cu) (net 19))
 (segment (start 191.77 78.74) (end 193.04 77.47) (width 0.381) (layer F.Cu) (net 22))
 (segment (start 200.66 77.47) (end 201.93 76.2) (width 0.381) (layer F.Cu) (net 22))
 (segment (start 193.04 77.47) (end 200.66 77.47) (width 0.381) (layer F.Cu) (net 22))
 (segment (start 194.31 78.74) (end 196.85 78.74) (width 0.381) (layer F.Cu) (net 20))
 (segment (start 203.2 97.79) (end 201.93 99.06) (width 0.381) (layer F.Cu) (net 20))
 (segment (start 203.2 80.645) (end 203.2 97.79) (width 0.381) (layer F.Cu) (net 20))
 (segment (start 202.565 80.01) (end 203.2 80.645) (width 0.381) (layer F.Cu) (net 20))
 (segment (start 198.12 80.01) (end 202.565 80.01) (width 0.381) (layer F.Cu) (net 20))
 (segment (start 196.85 78.74) (end 198.12 80.01) (width 0.381) (layer F.Cu) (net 20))
 (segment (start 184.15 93.98) (end 191.77 86.36) (width 0.381) (layer F.Cu) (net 26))
 (segment (start 191.77 86.36) (end 191.77 83.82) (width 0.381) (layer F.Cu) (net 26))
 (segment (start 191.77 81.28) (end 193.04 82.55) (width 0.381) (layer F.Cu) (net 21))
 (segment (start 197.485 89.535) (end 199.39 91.44) (width 0.381) (layer F.Cu) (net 21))
 (segment (start 197.485 83.82) (end 197.485 89.535) (width 0.381) (layer F.Cu) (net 21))
 (segment (start 196.215 82.55) (end 197.485 83.82) (width 0.381) (layer F.Cu) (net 21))
 (segment (start 193.04 82.55) (end 196.215 82.55) (width 0.381) (layer F.Cu) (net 21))
 (segment (start 199.39 96.52) (end 200.66 95.25) (width 0.381) (layer F.Cu) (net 23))
 (segment (start 196.85 81.28) (end 194.31 81.28) (width 0.381) (layer F.Cu) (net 23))
 (segment (start 198.12 82.55) (end 196.85 81.28) (width 0.381) (layer F.Cu) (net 23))
 (segment (start 200.025 82.55) (end 198.12 82.55) (width 0.381) (layer F.Cu) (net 23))
 (segment (start 200.66 83.185) (end 200.025 82.55) (width 0.381) (layer F.Cu) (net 23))
 (segment (start 200.66 95.25) (end 200.66 83.185) (width 0.381) (layer F.Cu) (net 23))
 (segment (start 194.31 83.82) (end 196.215 85.725) (width 0.381) (layer F.Cu) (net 24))
 (segment (start 196.215 90.805) (end 199.39 93.98) (width 0.381) (layer F.Cu) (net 24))
 (segment (start 196.215 85.725) (end 196.215 90.805) (width 0.381) (layer F.Cu) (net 24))
 (segment (start 184.15 96.52) (end 185.42 97.79) (width 0.381) (layer F.Cu) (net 25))
 (segment (start 198.12 97.79) (end 199.39 99.06) (width 0.381) (layer F.Cu) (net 25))
 (segment (start 185.42 97.79) (end 198.12 97.79) (width 0.381) (layer F.Cu) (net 25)))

